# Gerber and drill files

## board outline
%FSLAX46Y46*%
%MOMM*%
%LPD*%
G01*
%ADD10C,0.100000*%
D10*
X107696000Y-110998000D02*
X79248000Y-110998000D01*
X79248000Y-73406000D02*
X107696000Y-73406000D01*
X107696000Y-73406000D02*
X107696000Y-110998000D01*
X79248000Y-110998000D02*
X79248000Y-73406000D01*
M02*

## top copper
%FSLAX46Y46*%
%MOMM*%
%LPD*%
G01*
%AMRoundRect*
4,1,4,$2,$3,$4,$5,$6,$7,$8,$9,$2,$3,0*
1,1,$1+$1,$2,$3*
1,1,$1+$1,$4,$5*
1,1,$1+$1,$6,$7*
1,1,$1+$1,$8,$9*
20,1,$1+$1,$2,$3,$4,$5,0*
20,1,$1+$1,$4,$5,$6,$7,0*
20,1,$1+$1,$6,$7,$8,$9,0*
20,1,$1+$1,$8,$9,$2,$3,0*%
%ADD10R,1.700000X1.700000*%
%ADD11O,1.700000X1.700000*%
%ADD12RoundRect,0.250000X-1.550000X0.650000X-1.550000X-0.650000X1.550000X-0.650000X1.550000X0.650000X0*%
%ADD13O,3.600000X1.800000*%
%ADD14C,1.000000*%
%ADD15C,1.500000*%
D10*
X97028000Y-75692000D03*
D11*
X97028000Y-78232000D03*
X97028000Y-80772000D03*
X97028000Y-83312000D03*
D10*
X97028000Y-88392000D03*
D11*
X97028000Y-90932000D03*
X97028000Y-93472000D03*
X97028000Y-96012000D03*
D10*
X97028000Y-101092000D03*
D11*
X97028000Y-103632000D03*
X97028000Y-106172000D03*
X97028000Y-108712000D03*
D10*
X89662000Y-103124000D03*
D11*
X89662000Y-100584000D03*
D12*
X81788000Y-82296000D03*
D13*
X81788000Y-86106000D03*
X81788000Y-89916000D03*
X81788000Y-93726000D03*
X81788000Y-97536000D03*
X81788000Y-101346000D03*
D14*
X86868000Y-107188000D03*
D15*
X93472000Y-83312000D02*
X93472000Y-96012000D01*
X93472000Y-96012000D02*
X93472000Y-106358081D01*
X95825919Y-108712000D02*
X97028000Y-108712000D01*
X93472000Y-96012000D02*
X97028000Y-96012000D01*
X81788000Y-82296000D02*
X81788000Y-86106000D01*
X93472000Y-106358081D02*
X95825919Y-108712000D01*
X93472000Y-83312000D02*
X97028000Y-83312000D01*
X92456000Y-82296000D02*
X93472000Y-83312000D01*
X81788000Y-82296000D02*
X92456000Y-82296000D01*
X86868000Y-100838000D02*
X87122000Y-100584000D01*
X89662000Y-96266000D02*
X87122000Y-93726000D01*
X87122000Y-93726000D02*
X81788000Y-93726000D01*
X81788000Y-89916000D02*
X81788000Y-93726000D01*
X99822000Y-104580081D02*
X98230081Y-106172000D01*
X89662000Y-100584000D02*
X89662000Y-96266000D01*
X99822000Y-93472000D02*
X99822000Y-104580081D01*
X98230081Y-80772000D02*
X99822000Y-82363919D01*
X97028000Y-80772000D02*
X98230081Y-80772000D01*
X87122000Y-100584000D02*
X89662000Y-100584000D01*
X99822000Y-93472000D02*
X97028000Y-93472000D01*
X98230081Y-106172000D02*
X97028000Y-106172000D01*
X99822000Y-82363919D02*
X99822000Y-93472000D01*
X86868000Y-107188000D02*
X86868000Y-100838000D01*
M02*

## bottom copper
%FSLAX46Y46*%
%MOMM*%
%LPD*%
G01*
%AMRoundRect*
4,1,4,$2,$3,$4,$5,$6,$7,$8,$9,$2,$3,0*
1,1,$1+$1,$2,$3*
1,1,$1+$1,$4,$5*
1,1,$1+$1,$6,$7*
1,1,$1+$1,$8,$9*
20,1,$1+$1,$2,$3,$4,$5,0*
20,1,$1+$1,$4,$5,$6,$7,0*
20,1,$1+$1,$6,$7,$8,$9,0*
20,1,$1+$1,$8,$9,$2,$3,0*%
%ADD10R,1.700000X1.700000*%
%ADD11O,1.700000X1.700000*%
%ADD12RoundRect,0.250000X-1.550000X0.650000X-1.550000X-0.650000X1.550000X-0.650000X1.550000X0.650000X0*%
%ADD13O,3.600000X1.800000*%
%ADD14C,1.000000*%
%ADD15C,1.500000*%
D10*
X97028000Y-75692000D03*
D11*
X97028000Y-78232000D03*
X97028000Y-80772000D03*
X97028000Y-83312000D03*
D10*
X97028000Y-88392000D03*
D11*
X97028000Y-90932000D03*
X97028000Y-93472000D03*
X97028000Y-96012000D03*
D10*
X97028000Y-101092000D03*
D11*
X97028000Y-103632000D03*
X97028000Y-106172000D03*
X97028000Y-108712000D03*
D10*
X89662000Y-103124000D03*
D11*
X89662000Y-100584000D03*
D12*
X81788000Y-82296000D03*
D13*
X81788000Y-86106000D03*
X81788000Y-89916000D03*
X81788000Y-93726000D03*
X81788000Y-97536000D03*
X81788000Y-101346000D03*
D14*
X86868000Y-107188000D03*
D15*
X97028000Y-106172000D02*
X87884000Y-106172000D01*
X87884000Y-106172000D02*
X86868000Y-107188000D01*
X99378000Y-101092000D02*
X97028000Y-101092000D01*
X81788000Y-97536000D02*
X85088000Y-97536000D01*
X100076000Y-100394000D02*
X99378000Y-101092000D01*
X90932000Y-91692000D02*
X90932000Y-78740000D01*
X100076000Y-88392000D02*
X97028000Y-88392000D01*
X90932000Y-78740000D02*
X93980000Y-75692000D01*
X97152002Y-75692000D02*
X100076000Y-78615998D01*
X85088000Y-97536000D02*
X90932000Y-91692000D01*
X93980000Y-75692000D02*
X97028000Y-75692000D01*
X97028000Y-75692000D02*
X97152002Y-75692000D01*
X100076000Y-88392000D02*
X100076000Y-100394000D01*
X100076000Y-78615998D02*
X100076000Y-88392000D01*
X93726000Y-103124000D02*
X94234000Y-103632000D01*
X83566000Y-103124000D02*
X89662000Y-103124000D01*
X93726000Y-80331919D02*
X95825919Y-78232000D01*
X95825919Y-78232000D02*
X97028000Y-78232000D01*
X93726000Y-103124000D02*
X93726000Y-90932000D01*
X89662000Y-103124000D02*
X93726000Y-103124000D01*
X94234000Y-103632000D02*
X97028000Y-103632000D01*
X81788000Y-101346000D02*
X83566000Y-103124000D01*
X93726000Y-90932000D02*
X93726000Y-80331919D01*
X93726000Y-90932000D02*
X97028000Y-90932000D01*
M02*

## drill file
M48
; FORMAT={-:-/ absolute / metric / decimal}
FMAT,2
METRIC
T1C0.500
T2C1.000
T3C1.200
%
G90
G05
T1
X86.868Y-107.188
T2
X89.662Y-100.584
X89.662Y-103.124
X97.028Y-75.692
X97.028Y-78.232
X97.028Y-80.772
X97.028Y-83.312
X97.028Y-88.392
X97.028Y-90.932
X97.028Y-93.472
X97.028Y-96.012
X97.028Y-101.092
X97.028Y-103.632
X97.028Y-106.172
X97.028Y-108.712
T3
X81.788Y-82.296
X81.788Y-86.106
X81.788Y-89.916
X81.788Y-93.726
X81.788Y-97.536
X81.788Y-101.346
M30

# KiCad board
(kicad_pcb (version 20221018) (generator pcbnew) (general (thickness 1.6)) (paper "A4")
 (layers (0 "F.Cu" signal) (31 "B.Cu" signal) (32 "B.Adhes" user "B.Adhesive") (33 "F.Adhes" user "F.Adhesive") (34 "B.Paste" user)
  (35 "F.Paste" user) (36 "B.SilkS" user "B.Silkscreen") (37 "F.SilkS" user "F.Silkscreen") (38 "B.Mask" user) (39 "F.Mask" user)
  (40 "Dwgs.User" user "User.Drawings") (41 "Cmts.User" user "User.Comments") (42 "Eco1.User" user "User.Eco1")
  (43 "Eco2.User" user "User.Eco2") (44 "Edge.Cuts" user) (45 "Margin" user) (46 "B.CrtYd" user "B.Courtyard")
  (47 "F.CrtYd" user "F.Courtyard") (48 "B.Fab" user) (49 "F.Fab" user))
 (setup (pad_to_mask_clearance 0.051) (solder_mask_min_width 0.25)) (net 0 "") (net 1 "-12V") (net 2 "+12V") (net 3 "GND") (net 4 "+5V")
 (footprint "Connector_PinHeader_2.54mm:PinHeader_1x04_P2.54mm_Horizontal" (layer "F.Cu") (at 97.028 75.692)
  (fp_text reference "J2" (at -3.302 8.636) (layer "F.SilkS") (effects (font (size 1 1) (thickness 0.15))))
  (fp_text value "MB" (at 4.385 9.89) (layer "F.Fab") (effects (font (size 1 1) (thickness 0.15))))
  (pad "1" thru_hole rect (at 0 0) (size 1.7 1.7) (drill 1) (layers "*.Cu" "*.Mask") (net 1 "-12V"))
  (pad "2" thru_hole oval (at 0 2.54) (size 1.7 1.7) (drill 1) (layers "*.Cu" "*.Mask") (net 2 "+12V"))
  (pad "3" thru_hole oval (at 0 5.08) (size 1.7 1.7) (drill 1) (layers "*.Cu" "*.Mask") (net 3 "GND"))
  (pad "4" thru_hole oval (at 0 7.62) (size 1.7 1.7) (drill 1) (layers "*.Cu" "*.Mask") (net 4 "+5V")))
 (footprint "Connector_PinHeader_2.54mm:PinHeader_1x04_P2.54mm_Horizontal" (layer "F.Cu") (at 97.028 88.392)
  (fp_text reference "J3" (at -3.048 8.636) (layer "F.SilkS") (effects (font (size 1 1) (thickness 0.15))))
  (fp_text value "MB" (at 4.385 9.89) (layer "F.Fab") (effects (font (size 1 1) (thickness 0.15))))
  (pad "1" thru_hole rect (at 0 0) (size 1.7 1.7) (drill 1) (layers "*.Cu" "*.Mask") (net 1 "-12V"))
  (pad "2" thru_hole oval (at 0 2.54) (size 1.7 1.7) (drill 1) (layers "*.Cu" "*.Mask") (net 2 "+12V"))
  (pad "3" thru_hole oval (at 0 5.08) (size 1.7 1.7) (drill 1) (layers "*.Cu" "*.Mask") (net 3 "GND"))
  (pad "4" thru_hole oval (at 0 7.62) (size 1.7 1.7) (drill 1) (layers "*.Cu" "*.Mask") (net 4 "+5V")))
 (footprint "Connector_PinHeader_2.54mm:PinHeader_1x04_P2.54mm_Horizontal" (layer "F.Cu") (at 97.028 101.092)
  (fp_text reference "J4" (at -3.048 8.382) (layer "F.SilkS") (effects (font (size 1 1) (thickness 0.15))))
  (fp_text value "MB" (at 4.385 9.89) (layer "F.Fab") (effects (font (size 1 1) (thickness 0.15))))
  (pad "1" thru_hole rect (at 0 0) (size 1.7 1.7) (drill 1) (layers "*.Cu" "*.Mask") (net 1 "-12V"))
  (pad "2" thru_hole oval (at 0 2.54) (size 1.7 1.7) (drill 1) (layers "*.Cu" "*.Mask") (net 2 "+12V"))
  (pad "3" thru_hole oval (at 0 5.08) (size 1.7 1.7) (drill 1) (layers "*.Cu" "*.Mask") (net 3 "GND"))
  (pad "4" thru_hole oval (at 0 7.62) (size 1.7 1.7) (drill 1) (layers "*.Cu" "*.Mask") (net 4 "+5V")))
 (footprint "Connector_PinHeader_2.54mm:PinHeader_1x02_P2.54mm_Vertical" (layer "F.Cu") (at 89.662 103.124 180)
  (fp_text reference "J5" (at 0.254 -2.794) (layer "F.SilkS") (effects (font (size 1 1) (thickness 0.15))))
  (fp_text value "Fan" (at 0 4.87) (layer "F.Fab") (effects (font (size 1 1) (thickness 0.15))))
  (pad "1" thru_hole rect (at 0 0 180) (size 1.7 1.7) (drill 1) (layers "*.Cu" "*.Mask") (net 2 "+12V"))
  (pad "2" thru_hole oval (at 0 2.54 180) (size 1.7 1.7) (drill 1) (layers "*.Cu" "*.Mask") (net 3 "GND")))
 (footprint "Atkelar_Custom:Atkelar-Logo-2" (layer "F.Cu") (at 90.932 78.232)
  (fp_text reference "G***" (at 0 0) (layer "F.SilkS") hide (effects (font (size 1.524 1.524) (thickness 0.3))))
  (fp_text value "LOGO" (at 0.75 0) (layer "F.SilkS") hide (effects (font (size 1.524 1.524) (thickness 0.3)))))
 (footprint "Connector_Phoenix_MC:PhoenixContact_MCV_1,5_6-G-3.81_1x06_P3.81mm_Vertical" (layer "F.Cu") (at 81.788 82.296 -90)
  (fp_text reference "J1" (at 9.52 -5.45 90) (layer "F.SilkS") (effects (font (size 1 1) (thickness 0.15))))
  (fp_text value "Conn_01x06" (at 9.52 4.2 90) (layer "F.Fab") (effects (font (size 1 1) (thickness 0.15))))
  (pad "1" thru_hole roundrect (at 0 0 270) (size 1.8 3.6) (drill 1.2) (layers "*.Cu" "*.Mask") (roundrect_rratio 0.138889) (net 4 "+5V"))
  (pad "2" thru_hole oval (at 3.81 0 270) (size 1.8 3.6) (drill 1.2) (layers "*.Cu" "*.Mask") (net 4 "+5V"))
  (pad "3" thru_hole oval (at 7.62 0 270) (size 1.8 3.6) (drill 1.2) (layers "*.Cu" "*.Mask") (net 3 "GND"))
  (pad "4" thru_hole oval (at 11.43 0 270) (size 1.8 3.6) (drill 1.2) (layers "*.Cu" "*.Mask") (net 3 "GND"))
  (pad "5" thru_hole oval (at 15.24 0 270) (size 1.8 3.6) (drill 1.2) (layers "*.Cu" "*.Mask") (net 1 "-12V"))
  (pad "6" thru_hole oval (at 19.05 0 270) (size 1.8 3.6) (drill 1.2) (layers "*.Cu" "*.Mask") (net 2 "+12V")))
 (gr_line (start 107.696 110.998) (end 79.248 110.998) (stroke (width 0.1) (type solid)) (layer "Edge.Cuts"))
 (gr_line (start 79.248 73.406) (end 107.696 73.406) (stroke (width 0.1) (type solid)) (layer "Edge.Cuts"))
 (gr_line (start 107.696 73.406) (end 107.696 110.998) (stroke (width 0.1) (type solid)) (layer "Edge.Cuts"))
 (gr_line (start 79.248 110.998) (end 79.248 73.406) (stroke (width 0.1) (type solid)) (layer "Edge.Cuts"))
 (segment (start 93.472 83.312) (end 93.472 96.012) (width 1.5) (layer "F.Cu") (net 4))
 (segment (start 93.472 96.012) (end 93.472 106.358081) (width 1.5) (layer "F.Cu") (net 4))
 (segment (start 95.825919 108.712) (end 97.028 108.712) (width 1.5) (layer "F.Cu") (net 4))
 (segment (start 93.472 96.012) (end 97.028 96.012) (width 1.5) (layer "F.Cu") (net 4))
 (segment (start 81.788 82.296) (end 81.788 86.106) (width 1.5) (layer "F.Cu") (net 4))
 (segment (start 93.472 106.358081) (end 95.825919 108.712) (width 1.5) (layer "F.Cu") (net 4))
 (segment (start 93.472 83.312) (end 97.028 83.312) (width 1.5) (layer "F.Cu") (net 4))
 (segment (start 92.456 82.296) (end 93.472 83.312) (width 1.5) (layer "F.Cu") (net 4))
 (segment (start 81.788 82.296) (end 92.456 82.296) (width 1.5) (layer "F.Cu") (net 4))
 (segment (start 86.868 100.838) (end 87.122 100.584) (width 1.5) (layer "F.Cu") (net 3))
 (segment (start 89.662 96.266) (end 87.122 93.726) (width 1.5) (layer "F.Cu") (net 3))
 (segment (start 87.122 93.726) (end 81.788 93.726) (width 1.5) (layer "F.Cu") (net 3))
 (segment (start 81.788 89.916) (end 81.788 93.726) (width 1.5) (layer "F.Cu") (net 3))
 (segment (start 99.822 104.580081) (end 98.230081 106.172) (width 1.5) (layer "F.Cu") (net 3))
 (segment (start 89.662 100.584) (end 89.662 96.266) (width 1.5) (layer "F.Cu") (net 3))
 (segment (start 99.822 93.472) (end 99.822 104.580081) (width 1.5) (layer "F.Cu") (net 3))
 (segment (start 98.230081 80.772) (end 99.822 82.363919) (width 1.5) (layer "F.Cu") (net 3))
 (segment (start 97.028 80.772) (end 98.230081 80.772) (width 1.5) (layer "F.Cu") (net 3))
 (segment (start 87.122 100.584) (end 89.662 100.584) (width 1.5) (layer "F.Cu") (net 3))
 (segment (start 99.822 93.472) (end 97.028 93.472) (width 1.5) (layer "F.Cu") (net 3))
 (segment (start 98.230081 106.172) (end 97.028 106.172) (width 1.5) (layer "F.Cu") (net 3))
 (segment (start 99.822 82.363919) (end 99.822 93.472) (width 1.5) (layer "F.Cu") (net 3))
 (segment (start 86.868 107.188) (end 86.868 100.838) (width 1.5) (layer "F.Cu") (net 3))
 (via (at 86.868 107.188) (size 1) (drill 0.5) (layers "F.Cu" "B.Cu") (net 3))
 (segment (start 97.028 106.172) (end 87.884 106.172) (width 1.5) (layer "B.Cu") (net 3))
 (segment (start 87.884 106.172) (end 86.868 107.188) (width 1.5) (layer "B.Cu") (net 3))
 (segment (start 99.378 101.092) (end 97.028 101.092) (width 1.5) (layer "B.Cu") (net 1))
 (segment (start 81.788 97.536) (end 85.088 97.536) (width 1.5) (layer "B.Cu") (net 1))
 (segment (start 100.076 100.394) (end 99.378 101.092) (width 1.5) (layer "B.Cu") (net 1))
 (segment (start 90.932 91.692) (end 90.932 78.74) (width 1.5) (layer "B.Cu") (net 1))
 (segment (start 100.076 88.392) (end 97.028 88.392) (width 1.5) (layer "B.Cu") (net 1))
 (segment (start 90.932 78.74) (end 93.98 75.692) (width 1.5) (layer "B.Cu") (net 1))
 (segment (start 97.152002 75.692) (end 100.076 78.615998) (width 1.5) (layer "B.Cu") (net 1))
 (segment (start 85.088 97.536) (end 90.932 91.692) (width 1.5) (layer "B.Cu") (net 1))
 (segment (start 93.98 75.692) (end 97.028 75.692) (width 1.5) (layer "B.Cu") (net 1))
 (segment (start 97.028 75.692) (end 97.152002 75.692) (width 1.5) (layer "B.Cu") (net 1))
 (segment (start 100.076 88.392) (end 100.076 100.394) (width 1.5) (layer "B.Cu") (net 1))
 (segment (start 100.076 78.615998) (end 100.076 88.392) (width 1.5) (layer "B.Cu") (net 1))
 (segment (start 93.726 103.124) (end 94.234 103.632) (width 1.5) (layer "B.Cu") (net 2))
 (segment (start 83.566 103.124) (end 89.662 103.124) (width 1.5) (layer "B.Cu") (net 2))
 (segment (start 93.726 80.331919) (end 95.825919 78.232) (width 1.5) (layer "B.Cu") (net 2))
 (segment (start 95.825919 78.232) (end 97.028 78.232) (width 1.5) (layer "B.Cu") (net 2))
 (segment (start 93.726 103.124) (end 93.726 90.932) (width 1.5) (layer "B.Cu") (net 2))
 (segment (start 89.662 103.124) (end 93.726 103.124) (width 1.5) (layer "B.Cu") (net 2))
 (segment (start 94.234 103.632) (end 97.028 103.632) (width 1.5) (layer "B.Cu") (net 2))
 (segment (start 81.788 101.346) (end 83.566 103.124) (width 1.5) (layer "B.Cu") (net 2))
 (segment (start 93.726 90.932) (end 93.726 80.331919) (width 1.5) (layer "B.Cu") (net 2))
 (segment (start 93.726 90.932) (end 97.028 90.932) (width 1.5) (layer "B.Cu") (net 2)))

